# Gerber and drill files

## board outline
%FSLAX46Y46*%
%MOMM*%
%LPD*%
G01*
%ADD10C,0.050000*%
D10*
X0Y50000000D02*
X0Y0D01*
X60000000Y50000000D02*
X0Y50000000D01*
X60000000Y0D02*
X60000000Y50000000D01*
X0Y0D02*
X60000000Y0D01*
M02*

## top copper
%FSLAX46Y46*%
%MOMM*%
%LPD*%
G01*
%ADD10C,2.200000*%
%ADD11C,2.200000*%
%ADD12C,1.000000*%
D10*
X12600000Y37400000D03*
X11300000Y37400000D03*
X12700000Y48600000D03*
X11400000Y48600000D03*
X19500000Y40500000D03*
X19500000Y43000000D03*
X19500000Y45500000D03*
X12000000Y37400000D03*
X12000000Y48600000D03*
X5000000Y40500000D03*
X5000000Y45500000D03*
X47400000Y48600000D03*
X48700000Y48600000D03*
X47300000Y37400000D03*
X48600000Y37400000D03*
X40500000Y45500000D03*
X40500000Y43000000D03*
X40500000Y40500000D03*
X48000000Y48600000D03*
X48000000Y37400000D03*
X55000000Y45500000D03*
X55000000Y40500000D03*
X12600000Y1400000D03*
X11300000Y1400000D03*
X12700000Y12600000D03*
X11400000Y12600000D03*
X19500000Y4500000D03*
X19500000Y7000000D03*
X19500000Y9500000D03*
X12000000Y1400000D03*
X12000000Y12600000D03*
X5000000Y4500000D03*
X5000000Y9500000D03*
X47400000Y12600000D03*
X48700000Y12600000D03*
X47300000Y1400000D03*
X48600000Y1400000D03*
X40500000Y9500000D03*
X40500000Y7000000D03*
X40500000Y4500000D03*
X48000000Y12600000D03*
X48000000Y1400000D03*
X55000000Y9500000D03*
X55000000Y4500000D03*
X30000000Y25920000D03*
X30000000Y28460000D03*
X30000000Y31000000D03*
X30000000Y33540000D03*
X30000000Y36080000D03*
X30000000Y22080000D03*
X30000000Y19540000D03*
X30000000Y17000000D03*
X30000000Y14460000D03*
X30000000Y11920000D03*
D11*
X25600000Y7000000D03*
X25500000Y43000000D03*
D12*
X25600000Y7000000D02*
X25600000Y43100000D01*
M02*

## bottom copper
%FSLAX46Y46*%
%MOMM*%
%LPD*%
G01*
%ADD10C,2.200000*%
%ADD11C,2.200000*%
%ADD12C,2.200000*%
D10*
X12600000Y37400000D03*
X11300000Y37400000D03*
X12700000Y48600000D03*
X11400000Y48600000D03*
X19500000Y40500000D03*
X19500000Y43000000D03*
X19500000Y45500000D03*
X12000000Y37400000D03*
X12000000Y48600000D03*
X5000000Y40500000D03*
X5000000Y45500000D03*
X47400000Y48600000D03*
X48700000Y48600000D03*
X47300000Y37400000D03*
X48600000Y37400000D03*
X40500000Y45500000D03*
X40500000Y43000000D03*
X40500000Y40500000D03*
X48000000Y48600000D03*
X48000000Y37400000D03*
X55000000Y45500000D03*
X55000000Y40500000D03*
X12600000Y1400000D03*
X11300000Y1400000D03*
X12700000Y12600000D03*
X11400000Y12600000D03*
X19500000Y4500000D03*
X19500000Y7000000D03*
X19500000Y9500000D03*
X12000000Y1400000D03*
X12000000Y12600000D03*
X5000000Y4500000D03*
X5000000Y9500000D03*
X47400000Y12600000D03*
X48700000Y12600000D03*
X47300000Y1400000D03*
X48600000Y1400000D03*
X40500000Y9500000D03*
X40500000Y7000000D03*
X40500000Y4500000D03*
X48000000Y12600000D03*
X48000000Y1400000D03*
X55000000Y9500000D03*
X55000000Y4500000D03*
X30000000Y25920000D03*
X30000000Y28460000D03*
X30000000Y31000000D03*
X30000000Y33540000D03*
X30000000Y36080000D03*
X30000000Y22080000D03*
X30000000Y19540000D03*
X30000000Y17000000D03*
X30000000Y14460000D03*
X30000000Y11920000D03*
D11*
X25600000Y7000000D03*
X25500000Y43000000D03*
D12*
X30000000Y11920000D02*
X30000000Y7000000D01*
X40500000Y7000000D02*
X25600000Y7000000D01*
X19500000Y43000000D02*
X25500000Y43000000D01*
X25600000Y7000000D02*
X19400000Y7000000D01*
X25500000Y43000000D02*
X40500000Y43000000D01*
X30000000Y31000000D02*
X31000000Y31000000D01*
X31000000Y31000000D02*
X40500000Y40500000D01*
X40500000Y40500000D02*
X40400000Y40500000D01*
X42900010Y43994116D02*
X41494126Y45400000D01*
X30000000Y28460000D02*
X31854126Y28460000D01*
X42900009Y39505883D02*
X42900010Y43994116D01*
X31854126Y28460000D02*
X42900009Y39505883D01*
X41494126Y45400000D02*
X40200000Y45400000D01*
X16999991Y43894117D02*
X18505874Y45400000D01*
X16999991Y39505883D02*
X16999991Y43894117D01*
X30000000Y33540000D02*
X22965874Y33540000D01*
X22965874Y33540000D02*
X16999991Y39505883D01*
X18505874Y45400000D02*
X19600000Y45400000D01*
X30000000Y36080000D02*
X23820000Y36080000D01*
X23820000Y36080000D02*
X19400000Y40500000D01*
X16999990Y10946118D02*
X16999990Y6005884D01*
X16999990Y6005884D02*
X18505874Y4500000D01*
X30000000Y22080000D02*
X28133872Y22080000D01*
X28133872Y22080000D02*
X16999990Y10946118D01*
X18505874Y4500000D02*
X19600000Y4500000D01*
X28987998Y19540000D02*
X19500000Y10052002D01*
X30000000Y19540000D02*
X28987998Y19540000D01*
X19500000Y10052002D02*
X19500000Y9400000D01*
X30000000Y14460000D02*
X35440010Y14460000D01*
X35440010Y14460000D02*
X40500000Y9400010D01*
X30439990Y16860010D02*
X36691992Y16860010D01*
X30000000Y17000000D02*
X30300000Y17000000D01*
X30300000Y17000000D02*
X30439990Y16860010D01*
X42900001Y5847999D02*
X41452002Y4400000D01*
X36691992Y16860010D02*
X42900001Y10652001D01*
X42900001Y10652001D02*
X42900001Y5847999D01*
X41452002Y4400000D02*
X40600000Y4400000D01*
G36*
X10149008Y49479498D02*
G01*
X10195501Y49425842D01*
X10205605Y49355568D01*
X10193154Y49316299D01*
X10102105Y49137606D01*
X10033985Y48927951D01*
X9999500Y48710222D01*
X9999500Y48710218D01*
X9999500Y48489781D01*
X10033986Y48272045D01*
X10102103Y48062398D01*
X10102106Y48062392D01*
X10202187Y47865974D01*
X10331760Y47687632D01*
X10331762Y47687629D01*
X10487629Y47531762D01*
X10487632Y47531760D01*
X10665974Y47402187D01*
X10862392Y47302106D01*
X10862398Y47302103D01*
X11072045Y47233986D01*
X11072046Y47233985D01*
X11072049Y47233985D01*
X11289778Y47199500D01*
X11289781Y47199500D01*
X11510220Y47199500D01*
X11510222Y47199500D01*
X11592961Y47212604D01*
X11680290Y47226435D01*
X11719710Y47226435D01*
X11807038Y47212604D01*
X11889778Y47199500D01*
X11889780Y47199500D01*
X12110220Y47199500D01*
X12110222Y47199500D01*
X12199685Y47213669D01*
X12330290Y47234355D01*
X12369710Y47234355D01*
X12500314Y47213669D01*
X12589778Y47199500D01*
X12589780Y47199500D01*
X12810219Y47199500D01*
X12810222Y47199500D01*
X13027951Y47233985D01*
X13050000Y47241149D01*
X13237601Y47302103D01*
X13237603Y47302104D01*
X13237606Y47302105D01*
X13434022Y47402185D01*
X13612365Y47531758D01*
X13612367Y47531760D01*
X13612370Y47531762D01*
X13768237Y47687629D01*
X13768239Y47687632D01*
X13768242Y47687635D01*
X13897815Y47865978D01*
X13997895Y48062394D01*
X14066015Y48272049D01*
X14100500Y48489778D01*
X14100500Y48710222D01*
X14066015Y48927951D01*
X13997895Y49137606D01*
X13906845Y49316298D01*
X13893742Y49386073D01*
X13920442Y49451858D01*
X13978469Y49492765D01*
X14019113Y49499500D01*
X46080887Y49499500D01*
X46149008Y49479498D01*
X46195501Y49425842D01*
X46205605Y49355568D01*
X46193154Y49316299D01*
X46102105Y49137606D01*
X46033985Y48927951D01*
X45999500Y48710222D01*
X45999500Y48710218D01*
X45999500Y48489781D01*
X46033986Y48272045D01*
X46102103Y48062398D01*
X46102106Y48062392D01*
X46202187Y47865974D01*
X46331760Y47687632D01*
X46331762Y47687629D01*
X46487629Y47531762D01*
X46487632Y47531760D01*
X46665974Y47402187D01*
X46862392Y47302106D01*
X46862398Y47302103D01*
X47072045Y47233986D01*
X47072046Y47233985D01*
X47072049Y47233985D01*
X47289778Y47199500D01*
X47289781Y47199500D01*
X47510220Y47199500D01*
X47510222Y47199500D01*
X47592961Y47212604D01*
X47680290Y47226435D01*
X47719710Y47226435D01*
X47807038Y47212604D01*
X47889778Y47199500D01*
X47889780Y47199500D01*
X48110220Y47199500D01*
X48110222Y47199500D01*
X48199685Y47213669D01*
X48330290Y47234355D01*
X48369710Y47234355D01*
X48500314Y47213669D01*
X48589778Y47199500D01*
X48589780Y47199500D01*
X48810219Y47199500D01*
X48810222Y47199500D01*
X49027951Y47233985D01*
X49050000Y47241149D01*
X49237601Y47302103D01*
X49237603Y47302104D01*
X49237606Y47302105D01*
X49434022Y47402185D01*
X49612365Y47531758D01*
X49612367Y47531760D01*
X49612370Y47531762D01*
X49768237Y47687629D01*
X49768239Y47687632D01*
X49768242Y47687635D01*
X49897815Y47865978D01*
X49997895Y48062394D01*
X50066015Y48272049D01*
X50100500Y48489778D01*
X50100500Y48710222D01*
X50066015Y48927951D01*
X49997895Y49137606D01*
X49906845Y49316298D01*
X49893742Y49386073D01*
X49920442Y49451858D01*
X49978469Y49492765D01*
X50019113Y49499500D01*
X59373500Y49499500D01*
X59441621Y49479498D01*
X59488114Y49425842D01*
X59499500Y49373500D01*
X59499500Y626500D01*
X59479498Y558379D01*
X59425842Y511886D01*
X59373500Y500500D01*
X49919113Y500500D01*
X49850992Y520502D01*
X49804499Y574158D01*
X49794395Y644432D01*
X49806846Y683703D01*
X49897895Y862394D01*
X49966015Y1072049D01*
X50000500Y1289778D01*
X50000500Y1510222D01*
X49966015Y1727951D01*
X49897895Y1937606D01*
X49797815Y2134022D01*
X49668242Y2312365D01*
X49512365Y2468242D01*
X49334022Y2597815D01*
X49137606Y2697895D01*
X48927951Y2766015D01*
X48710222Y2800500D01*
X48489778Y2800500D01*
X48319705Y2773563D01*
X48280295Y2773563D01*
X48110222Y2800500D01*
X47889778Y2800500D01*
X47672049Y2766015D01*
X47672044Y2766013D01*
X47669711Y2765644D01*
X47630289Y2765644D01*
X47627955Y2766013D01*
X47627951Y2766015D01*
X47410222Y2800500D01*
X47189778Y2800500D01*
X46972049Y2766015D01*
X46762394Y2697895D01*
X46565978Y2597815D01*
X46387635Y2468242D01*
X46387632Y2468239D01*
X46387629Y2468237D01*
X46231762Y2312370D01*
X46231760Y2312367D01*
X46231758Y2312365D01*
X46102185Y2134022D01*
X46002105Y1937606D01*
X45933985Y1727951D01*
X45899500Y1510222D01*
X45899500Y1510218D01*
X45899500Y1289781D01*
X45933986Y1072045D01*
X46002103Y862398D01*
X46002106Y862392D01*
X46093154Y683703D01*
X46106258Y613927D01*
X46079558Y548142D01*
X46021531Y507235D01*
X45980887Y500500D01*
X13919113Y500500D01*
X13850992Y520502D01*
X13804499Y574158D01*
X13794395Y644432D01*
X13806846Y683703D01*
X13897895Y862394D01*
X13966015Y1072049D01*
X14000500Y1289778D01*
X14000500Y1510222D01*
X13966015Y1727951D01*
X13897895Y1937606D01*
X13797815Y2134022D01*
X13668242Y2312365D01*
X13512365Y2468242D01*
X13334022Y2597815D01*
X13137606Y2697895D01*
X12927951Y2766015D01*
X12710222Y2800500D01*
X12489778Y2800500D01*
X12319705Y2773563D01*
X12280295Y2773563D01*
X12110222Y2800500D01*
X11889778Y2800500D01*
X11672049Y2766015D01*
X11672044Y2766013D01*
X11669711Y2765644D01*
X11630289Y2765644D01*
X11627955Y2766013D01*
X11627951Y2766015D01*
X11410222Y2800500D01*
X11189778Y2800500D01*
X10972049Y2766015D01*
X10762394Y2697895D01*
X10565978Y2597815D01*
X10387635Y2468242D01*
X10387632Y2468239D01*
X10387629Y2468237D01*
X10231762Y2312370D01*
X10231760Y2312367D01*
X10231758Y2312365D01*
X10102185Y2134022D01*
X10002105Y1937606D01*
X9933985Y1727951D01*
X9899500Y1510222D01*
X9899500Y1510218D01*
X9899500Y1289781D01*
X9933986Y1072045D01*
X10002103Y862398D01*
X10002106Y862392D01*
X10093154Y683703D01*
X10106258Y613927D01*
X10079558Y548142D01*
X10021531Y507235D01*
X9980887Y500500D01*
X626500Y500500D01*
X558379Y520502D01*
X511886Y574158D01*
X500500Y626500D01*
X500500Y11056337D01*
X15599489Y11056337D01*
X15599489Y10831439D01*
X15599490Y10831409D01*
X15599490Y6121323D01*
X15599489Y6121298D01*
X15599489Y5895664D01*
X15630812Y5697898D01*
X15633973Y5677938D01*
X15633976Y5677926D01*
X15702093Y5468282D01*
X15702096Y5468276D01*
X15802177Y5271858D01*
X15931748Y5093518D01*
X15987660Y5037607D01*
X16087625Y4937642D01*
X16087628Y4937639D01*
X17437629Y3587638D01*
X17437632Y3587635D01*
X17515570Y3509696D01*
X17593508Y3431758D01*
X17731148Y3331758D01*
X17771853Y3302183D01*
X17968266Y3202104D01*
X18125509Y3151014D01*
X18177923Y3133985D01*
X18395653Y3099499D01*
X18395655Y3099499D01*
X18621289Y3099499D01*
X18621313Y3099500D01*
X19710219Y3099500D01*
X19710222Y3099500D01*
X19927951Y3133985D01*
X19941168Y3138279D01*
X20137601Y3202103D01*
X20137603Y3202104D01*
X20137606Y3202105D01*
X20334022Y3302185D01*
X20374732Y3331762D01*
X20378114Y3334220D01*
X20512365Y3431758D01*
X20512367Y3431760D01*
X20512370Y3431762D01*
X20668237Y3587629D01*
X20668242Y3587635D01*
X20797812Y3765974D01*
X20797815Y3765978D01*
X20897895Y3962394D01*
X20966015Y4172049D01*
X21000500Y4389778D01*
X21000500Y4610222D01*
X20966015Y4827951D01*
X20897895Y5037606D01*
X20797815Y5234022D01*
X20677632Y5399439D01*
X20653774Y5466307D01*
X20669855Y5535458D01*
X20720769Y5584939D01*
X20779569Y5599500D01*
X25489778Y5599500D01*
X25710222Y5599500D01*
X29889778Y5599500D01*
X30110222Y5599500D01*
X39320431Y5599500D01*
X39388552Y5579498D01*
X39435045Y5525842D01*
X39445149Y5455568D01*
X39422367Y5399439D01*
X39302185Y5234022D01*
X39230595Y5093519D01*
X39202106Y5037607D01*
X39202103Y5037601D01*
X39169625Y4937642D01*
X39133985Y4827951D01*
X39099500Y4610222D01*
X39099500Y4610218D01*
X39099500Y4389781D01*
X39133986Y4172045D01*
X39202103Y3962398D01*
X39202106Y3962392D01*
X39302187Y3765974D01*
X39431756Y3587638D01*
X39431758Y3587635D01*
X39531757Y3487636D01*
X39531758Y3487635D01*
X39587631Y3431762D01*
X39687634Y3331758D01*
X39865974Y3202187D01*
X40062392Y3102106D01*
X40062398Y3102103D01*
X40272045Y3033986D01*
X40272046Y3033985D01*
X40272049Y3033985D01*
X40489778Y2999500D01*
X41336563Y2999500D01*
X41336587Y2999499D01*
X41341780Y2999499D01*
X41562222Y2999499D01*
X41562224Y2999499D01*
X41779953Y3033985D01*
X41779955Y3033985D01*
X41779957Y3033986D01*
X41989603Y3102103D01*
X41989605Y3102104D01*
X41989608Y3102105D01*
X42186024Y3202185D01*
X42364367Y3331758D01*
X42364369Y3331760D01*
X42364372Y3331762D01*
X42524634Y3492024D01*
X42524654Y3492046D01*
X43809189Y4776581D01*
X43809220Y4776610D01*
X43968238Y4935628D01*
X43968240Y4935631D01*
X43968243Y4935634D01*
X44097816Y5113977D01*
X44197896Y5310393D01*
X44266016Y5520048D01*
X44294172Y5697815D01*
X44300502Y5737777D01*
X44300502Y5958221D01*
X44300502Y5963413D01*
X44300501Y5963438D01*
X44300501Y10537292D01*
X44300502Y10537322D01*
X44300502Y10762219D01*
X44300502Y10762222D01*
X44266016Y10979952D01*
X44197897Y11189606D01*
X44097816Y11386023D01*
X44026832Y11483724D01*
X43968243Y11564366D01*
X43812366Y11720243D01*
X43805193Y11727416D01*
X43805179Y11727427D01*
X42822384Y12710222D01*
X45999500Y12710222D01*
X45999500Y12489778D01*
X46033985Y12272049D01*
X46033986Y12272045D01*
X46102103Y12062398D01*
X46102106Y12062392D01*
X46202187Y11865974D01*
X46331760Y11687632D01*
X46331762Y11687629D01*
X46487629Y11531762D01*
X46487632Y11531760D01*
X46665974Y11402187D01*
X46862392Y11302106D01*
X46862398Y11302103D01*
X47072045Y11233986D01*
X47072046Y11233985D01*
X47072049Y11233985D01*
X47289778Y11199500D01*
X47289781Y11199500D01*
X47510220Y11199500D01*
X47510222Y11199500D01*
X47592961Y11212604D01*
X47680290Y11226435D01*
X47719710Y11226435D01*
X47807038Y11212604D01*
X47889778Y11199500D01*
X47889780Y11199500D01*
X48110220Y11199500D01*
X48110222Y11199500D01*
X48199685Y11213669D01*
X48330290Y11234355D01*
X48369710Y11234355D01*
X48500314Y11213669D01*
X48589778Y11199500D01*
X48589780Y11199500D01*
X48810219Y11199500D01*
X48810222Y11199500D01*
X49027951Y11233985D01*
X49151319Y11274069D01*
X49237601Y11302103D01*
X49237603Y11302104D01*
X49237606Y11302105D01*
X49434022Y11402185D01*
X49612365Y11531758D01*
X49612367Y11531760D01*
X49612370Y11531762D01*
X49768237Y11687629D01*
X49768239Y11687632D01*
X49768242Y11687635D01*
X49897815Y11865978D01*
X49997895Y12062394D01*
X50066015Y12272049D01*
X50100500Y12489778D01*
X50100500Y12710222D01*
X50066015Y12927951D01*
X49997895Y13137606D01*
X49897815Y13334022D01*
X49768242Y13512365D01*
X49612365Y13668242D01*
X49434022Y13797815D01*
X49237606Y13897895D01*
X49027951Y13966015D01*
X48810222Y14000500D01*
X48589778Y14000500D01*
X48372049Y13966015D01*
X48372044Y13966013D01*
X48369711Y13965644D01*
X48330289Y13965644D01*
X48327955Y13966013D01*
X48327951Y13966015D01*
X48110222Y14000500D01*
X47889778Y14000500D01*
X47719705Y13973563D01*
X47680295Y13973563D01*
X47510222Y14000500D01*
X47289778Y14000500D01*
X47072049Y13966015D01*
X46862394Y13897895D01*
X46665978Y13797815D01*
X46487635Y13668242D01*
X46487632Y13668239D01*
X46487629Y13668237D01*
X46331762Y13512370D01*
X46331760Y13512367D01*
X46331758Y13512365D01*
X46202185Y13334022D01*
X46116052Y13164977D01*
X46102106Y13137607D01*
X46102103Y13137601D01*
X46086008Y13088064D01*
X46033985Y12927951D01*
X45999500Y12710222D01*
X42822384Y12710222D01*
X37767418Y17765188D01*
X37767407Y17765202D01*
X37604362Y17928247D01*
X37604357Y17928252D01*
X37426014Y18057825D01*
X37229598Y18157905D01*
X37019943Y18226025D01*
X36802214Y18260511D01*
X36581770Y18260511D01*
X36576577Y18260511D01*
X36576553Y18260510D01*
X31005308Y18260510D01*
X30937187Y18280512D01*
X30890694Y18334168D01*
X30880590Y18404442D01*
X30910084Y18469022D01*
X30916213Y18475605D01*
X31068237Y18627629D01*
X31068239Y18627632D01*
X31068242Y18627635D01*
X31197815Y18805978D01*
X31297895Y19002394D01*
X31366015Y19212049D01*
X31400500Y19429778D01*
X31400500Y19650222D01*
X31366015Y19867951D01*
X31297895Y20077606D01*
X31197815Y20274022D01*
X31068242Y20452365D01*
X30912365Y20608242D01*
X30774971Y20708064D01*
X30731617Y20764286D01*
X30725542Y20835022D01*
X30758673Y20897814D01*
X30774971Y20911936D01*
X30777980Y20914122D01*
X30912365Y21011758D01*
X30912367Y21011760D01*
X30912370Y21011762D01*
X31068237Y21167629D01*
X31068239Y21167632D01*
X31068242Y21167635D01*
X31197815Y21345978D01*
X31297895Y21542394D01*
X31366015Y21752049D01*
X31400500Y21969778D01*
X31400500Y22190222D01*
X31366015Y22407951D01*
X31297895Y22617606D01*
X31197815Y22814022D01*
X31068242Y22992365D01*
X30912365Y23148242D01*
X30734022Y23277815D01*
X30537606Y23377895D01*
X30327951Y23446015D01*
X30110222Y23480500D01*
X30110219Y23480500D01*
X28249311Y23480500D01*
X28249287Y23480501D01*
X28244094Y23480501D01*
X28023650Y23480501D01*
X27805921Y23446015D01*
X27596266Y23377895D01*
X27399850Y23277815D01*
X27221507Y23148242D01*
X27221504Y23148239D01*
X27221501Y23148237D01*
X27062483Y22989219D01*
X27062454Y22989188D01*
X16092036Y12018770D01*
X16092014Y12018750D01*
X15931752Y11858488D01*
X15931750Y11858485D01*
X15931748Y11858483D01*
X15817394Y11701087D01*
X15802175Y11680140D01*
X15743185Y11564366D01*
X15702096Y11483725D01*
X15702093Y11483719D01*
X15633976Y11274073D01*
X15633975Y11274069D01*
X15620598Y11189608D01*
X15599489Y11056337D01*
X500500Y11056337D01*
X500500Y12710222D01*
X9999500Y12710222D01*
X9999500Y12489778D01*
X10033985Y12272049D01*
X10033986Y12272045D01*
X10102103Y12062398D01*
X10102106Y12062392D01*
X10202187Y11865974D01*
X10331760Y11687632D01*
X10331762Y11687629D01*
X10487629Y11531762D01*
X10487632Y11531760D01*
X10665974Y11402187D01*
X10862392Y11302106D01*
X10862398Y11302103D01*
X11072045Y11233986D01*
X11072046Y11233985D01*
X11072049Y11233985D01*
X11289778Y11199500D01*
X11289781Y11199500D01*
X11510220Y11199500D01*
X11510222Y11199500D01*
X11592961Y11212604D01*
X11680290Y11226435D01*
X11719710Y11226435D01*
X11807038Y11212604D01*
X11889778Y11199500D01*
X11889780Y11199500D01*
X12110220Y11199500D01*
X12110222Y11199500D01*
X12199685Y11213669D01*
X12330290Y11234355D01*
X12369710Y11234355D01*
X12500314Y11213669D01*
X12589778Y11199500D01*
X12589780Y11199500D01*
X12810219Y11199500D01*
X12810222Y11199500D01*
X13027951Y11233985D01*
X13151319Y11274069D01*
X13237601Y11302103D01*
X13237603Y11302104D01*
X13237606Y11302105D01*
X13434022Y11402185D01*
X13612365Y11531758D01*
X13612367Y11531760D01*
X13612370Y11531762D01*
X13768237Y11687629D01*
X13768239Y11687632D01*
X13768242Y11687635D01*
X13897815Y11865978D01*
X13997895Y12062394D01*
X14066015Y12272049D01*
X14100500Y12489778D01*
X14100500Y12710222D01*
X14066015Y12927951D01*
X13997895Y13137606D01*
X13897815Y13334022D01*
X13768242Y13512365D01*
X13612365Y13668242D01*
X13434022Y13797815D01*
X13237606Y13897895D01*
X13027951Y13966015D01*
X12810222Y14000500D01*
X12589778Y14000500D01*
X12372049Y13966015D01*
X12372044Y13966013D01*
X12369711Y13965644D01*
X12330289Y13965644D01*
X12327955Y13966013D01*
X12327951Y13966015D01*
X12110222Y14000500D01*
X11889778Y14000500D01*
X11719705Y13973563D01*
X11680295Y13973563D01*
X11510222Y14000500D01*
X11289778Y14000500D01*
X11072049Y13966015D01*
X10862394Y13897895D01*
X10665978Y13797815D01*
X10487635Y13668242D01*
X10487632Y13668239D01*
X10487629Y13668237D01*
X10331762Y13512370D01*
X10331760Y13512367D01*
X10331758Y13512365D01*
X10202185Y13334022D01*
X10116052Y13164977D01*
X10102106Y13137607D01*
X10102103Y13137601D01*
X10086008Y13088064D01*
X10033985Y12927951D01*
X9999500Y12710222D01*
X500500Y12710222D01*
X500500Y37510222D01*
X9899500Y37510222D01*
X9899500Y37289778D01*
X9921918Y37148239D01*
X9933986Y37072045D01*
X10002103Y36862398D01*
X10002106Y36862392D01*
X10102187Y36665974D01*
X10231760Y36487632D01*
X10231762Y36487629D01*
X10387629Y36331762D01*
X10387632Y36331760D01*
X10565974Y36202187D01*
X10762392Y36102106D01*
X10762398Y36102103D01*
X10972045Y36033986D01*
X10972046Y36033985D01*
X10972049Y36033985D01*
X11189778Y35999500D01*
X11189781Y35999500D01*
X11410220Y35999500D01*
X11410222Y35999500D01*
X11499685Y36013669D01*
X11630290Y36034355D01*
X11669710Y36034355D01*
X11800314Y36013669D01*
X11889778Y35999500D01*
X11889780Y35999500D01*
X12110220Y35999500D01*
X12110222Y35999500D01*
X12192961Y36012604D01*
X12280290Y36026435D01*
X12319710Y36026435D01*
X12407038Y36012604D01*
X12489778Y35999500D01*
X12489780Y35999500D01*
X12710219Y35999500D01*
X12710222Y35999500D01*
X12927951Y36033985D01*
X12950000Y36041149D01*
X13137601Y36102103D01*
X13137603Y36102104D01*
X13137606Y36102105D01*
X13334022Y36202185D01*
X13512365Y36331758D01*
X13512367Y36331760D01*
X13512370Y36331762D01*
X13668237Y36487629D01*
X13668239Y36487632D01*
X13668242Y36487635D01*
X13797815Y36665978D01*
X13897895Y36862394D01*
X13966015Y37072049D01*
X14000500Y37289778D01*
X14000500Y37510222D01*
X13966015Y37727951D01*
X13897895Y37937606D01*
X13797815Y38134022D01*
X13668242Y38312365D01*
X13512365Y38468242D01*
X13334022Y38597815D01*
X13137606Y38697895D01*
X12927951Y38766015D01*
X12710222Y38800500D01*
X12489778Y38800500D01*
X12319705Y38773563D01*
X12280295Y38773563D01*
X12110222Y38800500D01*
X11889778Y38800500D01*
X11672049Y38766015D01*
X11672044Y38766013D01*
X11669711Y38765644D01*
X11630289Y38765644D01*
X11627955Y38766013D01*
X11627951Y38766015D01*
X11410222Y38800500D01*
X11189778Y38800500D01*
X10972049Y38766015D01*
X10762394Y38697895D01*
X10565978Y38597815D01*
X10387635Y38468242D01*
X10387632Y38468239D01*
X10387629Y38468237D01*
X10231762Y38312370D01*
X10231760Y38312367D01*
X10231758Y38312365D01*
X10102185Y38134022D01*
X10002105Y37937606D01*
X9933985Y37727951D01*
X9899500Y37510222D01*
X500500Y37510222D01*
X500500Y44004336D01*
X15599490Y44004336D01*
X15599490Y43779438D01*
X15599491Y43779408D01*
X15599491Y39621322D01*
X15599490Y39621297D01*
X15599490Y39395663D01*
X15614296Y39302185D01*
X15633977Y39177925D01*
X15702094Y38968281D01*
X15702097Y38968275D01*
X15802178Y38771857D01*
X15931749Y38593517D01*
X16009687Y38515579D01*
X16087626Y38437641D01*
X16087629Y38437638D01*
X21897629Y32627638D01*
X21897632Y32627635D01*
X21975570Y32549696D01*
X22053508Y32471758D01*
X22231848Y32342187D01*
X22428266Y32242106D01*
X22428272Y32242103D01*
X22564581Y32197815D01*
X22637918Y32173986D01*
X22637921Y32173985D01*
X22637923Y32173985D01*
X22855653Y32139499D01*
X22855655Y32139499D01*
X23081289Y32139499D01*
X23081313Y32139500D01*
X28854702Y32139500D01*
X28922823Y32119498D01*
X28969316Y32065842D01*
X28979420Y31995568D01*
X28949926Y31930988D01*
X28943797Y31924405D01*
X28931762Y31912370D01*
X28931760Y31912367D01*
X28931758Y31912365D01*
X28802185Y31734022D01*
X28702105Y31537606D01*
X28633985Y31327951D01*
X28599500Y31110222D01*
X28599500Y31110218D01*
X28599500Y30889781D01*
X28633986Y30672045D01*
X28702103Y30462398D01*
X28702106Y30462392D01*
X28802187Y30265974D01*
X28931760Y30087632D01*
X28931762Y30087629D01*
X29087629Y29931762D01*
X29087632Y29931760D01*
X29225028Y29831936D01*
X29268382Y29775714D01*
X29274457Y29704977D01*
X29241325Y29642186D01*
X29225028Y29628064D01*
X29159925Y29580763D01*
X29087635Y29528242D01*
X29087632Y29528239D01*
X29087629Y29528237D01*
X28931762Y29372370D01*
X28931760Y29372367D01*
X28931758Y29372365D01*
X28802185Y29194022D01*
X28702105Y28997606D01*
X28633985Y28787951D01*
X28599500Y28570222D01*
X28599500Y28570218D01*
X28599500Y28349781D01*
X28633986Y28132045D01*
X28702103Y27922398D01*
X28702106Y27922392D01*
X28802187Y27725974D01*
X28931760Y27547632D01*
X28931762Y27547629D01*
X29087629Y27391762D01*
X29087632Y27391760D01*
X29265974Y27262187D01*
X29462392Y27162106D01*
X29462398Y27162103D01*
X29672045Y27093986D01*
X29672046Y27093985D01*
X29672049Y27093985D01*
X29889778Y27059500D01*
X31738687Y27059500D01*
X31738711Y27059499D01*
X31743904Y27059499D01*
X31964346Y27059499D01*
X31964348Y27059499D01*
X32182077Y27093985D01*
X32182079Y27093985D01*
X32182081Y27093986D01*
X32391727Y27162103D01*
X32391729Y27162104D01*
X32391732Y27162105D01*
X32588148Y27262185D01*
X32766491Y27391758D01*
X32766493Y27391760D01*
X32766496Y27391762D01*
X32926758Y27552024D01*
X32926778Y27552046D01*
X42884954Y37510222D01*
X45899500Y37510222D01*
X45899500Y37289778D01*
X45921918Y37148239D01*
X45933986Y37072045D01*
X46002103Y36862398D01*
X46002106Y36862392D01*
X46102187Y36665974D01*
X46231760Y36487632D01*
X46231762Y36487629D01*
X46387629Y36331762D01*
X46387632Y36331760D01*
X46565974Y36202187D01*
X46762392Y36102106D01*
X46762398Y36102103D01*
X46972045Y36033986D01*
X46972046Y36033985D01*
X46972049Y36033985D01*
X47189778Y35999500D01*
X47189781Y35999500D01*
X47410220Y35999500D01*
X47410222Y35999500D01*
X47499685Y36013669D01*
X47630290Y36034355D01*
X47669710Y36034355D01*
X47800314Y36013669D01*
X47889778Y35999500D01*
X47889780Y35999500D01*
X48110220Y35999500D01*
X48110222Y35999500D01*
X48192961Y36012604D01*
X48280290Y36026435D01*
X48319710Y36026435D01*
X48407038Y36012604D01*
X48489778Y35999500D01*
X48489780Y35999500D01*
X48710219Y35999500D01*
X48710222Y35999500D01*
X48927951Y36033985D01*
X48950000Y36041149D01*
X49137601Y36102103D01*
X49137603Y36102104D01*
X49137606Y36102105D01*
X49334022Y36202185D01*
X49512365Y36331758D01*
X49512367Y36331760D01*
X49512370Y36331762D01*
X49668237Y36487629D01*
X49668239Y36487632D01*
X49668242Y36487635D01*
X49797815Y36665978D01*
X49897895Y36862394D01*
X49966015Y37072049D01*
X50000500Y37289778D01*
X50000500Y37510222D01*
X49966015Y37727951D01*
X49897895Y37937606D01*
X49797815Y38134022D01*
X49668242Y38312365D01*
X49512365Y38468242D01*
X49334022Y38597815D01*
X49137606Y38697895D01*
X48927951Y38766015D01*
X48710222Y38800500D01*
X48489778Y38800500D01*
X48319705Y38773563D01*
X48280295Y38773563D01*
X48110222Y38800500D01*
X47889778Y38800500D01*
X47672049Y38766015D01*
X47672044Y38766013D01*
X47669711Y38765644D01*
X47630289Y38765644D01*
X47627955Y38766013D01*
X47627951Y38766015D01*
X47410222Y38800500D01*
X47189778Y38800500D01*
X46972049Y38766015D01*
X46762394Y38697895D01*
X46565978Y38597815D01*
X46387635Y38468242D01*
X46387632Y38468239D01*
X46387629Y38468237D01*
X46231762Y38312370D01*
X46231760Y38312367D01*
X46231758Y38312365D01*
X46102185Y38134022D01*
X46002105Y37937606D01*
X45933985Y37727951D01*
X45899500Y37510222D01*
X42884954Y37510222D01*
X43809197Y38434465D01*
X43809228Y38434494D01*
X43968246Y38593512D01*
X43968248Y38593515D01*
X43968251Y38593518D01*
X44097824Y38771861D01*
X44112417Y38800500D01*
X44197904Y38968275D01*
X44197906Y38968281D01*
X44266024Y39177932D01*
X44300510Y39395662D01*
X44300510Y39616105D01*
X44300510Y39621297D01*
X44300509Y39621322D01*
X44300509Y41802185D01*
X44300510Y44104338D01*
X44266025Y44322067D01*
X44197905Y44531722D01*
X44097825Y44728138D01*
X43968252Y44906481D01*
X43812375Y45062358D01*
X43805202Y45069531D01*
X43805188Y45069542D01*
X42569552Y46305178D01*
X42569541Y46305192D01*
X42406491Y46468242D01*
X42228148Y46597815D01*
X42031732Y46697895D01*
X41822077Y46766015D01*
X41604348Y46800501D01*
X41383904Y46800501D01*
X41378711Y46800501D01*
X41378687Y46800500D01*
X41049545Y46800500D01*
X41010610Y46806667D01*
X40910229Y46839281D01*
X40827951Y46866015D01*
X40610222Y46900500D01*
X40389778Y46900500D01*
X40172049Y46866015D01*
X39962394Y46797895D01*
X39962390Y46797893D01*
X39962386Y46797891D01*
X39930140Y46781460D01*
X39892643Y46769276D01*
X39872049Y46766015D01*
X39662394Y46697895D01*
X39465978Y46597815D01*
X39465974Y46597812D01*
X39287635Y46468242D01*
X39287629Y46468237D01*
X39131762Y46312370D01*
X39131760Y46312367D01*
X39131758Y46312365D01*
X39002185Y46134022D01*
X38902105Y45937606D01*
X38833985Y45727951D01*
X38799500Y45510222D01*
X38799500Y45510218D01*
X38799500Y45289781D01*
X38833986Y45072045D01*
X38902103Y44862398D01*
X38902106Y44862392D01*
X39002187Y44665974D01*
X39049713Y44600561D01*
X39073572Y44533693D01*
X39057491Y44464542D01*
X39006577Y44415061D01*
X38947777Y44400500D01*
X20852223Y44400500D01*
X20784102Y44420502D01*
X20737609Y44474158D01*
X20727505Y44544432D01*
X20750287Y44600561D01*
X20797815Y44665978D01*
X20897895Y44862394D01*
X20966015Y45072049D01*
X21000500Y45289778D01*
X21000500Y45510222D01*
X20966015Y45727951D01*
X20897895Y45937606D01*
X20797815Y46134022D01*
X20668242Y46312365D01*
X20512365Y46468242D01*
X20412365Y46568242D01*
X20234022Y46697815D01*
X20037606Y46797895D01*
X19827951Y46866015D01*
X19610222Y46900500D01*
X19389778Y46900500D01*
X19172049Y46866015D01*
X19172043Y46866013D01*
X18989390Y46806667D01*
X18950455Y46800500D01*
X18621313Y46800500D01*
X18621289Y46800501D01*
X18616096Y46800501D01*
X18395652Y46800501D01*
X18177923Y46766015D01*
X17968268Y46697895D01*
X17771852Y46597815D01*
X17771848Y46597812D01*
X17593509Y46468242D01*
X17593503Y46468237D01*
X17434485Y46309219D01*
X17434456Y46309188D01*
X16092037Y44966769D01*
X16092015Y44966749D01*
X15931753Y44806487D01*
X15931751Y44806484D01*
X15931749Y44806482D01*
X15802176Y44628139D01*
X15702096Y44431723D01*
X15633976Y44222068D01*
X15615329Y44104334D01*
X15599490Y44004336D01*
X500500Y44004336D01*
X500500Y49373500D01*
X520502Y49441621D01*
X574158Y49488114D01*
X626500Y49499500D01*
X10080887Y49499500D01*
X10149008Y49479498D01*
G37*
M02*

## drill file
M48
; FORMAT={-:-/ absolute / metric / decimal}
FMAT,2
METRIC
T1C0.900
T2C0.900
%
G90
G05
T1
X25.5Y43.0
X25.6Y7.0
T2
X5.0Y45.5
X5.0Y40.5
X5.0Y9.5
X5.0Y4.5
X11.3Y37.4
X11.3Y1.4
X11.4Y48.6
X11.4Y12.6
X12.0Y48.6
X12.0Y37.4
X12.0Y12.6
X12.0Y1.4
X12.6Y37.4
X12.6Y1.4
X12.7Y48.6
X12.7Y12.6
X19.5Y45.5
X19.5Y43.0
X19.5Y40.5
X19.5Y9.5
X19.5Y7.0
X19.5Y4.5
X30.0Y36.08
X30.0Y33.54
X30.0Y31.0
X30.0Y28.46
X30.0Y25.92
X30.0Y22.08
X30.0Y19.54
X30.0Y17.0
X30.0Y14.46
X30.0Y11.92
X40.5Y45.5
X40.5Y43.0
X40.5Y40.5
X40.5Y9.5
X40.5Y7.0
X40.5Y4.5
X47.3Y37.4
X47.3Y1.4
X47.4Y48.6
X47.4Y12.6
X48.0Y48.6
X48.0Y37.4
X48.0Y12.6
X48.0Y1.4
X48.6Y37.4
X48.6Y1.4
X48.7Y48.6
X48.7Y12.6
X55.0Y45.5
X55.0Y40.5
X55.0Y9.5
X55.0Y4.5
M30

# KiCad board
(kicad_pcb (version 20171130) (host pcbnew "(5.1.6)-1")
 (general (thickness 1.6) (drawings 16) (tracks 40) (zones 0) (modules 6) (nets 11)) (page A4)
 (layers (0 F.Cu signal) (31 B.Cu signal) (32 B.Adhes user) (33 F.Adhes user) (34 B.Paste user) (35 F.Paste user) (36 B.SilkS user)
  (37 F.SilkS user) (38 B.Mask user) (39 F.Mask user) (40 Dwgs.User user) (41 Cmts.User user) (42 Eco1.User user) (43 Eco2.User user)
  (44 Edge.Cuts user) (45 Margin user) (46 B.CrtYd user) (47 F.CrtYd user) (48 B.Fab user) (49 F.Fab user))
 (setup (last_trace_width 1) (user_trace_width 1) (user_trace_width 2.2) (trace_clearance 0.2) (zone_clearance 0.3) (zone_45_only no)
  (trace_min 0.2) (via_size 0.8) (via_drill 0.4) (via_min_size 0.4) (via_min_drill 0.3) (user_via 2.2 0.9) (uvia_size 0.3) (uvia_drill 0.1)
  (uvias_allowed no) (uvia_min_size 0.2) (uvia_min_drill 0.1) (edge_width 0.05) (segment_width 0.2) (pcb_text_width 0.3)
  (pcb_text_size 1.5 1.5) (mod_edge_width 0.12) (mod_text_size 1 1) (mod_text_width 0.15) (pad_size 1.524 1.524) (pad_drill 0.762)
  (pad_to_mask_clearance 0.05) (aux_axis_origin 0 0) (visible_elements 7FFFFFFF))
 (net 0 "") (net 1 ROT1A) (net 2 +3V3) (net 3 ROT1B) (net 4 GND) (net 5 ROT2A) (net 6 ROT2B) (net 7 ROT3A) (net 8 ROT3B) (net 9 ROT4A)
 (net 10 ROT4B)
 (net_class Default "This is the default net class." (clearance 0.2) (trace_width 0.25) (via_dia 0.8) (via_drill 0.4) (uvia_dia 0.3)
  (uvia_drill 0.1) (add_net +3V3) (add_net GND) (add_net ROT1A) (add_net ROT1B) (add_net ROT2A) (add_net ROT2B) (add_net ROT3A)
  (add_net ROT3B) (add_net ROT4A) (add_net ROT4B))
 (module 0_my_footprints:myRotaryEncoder (layer F.Cu) (at 12 -43 180)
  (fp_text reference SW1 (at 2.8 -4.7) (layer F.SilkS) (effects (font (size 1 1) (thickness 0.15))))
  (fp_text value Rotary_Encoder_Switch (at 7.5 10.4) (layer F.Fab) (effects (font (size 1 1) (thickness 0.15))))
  (pad "" thru_hole circle (at -0.6 -5.6 180) (size 2.2 2.2) (drill 0.9) (layers *.Cu *.Mask))
  (pad "" thru_hole circle (at 0.7 -5.6 180) (size 2.2 2.2) (drill 0.9) (layers *.Cu *.Mask))
  (pad "" thru_hole circle (at -0.7 5.6 180) (size 2.2 2.2) (drill 0.9) (layers *.Cu *.Mask))
  (pad "" thru_hole circle (at 0.6 5.6 180) (size 2.2 2.2) (drill 0.9) (layers *.Cu *.Mask))
  (pad A thru_hole circle (at -7.5 -2.5 180) (size 2.2 2.2) (drill 0.9) (layers *.Cu *.Mask) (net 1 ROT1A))
  (pad C thru_hole circle (at -7.5 0 180) (size 2.2 2.2) (drill 0.9) (layers *.Cu *.Mask) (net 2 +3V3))
  (pad B thru_hole circle (at -7.5 2.5 180) (size 2.2 2.2) (drill 0.9) (layers *.Cu *.Mask) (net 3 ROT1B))
  (pad "" thru_hole circle (at 0 -5.6 180) (size 2.2 2.2) (drill 0.9) (layers *.Cu *.Mask))
  (pad "" thru_hole circle (at 0 5.6 180) (size 2.2 2.2) (drill 0.9) (layers *.Cu *.Mask))
  (pad S1 thru_hole circle (at 7 -2.5 180) (size 2.2 2.2) (drill 0.9) (layers *.Cu *.Mask) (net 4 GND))
  (pad S2 thru_hole circle (at 7 2.5 180) (size 2.2 2.2) (drill 0.9) (layers *.Cu *.Mask) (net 4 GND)))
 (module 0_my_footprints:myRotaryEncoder (layer F.Cu) (at 48 -43)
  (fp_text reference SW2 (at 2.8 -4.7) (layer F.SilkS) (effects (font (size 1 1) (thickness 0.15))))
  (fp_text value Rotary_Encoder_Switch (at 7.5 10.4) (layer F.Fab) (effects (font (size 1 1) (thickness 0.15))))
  (pad "" thru_hole circle (at -0.6 -5.6) (size 2.2 2.2) (drill 0.9) (layers *.Cu *.Mask))
  (pad "" thru_hole circle (at 0.7 -5.6) (size 2.2 2.2) (drill 0.9) (layers *.Cu *.Mask))
  (pad "" thru_hole circle (at -0.7 5.6) (size 2.2 2.2) (drill 0.9) (layers *.Cu *.Mask))
  (pad "" thru_hole circle (at 0.6 5.6) (size 2.2 2.2) (drill 0.9) (layers *.Cu *.Mask))
  (pad A thru_hole circle (at -7.5 -2.5) (size 2.2 2.2) (drill 0.9) (layers *.Cu *.Mask) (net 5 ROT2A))
  (pad C thru_hole circle (at -7.5 0) (size 2.2 2.2) (drill 0.9) (layers *.Cu *.Mask) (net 2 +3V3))
  (pad B thru_hole circle (at -7.5 2.5) (size 2.2 2.2) (drill 0.9) (layers *.Cu *.Mask) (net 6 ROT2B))
  (pad "" thru_hole circle (at 0 -5.6) (size 2.2 2.2) (drill 0.9) (layers *.Cu *.Mask))
  (pad "" thru_hole circle (at 0 5.6) (size 2.2 2.2) (drill 0.9) (layers *.Cu *.Mask))
  (pad S1 thru_hole circle (at 7 -2.5) (size 2.2 2.2) (drill 0.9) (layers *.Cu *.Mask) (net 4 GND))
  (pad S2 thru_hole circle (at 7 2.5) (size 2.2 2.2) (drill 0.9) (layers *.Cu *.Mask) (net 4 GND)))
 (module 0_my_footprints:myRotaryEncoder (layer F.Cu) (at 12 -7 180)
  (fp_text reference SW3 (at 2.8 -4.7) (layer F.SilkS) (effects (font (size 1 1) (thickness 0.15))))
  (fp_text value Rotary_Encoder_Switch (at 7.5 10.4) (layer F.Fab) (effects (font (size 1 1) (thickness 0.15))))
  (pad "" thru_hole circle (at -0.6 -5.6 180) (size 2.2 2.2) (drill 0.9) (layers *.Cu *.Mask))
  (pad "" thru_hole circle (at 0.7 -5.6 180) (size 2.2 2.2) (drill 0.9) (layers *.Cu *.Mask))
  (pad "" thru_hole circle (at -0.7 5.6 180) (size 2.2 2.2) (drill 0.9) (layers *.Cu *.Mask))
  (pad "" thru_hole circle (at 0.6 5.6 180) (size 2.2 2.2) (drill 0.9) (layers *.Cu *.Mask))
  (pad A thru_hole circle (at -7.5 -2.5 180) (size 2.2 2.2) (drill 0.9) (layers *.Cu *.Mask) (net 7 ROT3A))
  (pad C thru_hole circle (at -7.5 0 180) (size 2.2 2.2) (drill 0.9) (layers *.Cu *.Mask) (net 2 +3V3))
  (pad B thru_hole circle (at -7.5 2.5 180) (size 2.2 2.2) (drill 0.9) (layers *.Cu *.Mask) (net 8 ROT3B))
  (pad "" thru_hole circle (at 0 -5.6 180) (size 2.2 2.2) (drill 0.9) (layers *.Cu *.Mask))
  (pad "" thru_hole circle (at 0 5.6 180) (size 2.2 2.2) (drill 0.9) (layers *.Cu *.Mask))
  (pad S1 thru_hole circle (at 7 -2.5 180) (size 2.2 2.2) (drill 0.9) (layers *.Cu *.Mask) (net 4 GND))
  (pad S2 thru_hole circle (at 7 2.5 180) (size 2.2 2.2) (drill 0.9) (layers *.Cu *.Mask) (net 4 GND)))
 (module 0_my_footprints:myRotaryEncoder (layer F.Cu) (at 48 -7)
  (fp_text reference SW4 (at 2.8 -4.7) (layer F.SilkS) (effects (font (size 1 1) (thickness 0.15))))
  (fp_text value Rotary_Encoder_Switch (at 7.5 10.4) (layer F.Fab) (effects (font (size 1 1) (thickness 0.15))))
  (pad "" thru_hole circle (at -0.6 -5.6) (size 2.2 2.2) (drill 0.9) (layers *.Cu *.Mask))
  (pad "" thru_hole circle (at 0.7 -5.6) (size 2.2 2.2) (drill 0.9) (layers *.Cu *.Mask))
  (pad "" thru_hole circle (at -0.7 5.6) (size 2.2 2.2) (drill 0.9) (layers *.Cu *.Mask))
  (pad "" thru_hole circle (at 0.6 5.6) (size 2.2 2.2) (drill 0.9) (layers *.Cu *.Mask))
  (pad A thru_hole circle (at -7.5 -2.5) (size 2.2 2.2) (drill 0.9) (layers *.Cu *.Mask) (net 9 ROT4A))
  (pad C thru_hole circle (at -7.5 0) (size 2.2 2.2) (drill 0.9) (layers *.Cu *.Mask) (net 2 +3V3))
  (pad B thru_hole circle (at -7.5 2.5) (size 2.2 2.2) (drill 0.9) (layers *.Cu *.Mask) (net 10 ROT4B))
  (pad "" thru_hole circle (at 0 -5.6) (size 2.2 2.2) (drill 0.9) (layers *.Cu *.Mask))
  (pad "" thru_hole circle (at 0 5.6) (size 2.2 2.2) (drill 0.9) (layers *.Cu *.Mask))
  (pad S1 thru_hole circle (at 7 -2.5) (size 2.2 2.2) (drill 0.9) (layers *.Cu *.Mask) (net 4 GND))
  (pad S2 thru_hole circle (at 7 2.5) (size 2.2 2.2) (drill 0.9) (layers *.Cu *.Mask) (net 4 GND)))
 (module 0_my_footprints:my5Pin (layer F.Cu) (at 30 -31 270)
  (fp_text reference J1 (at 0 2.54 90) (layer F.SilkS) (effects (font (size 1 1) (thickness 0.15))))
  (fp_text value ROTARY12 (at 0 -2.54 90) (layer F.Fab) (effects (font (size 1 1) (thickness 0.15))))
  (pad 5 thru_hole circle (at 5.08 0 270) (size 2.2 2.2) (drill 0.9) (layers *.Cu *.Mask) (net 4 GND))
  (pad 4 thru_hole circle (at 2.54 0 270) (size 2.2 2.2) (drill 0.9) (layers *.Cu *.Mask) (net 5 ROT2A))
  (pad 3 thru_hole circle (at 0 0 270) (size 2.2 2.2) (drill 0.9) (layers *.Cu *.Mask) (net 6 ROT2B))
  (pad 2 thru_hole circle (at -2.54 0 270) (size 2.2 2.2) (drill 0.9) (layers *.Cu *.Mask) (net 3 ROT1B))
  (pad 1 thru_hole circle (at -5.08 0 270) (size 2.2 2.2) (drill 0.9) (layers *.Cu *.Mask) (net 1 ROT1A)))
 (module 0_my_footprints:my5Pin (layer F.Cu) (at 30 -17 270)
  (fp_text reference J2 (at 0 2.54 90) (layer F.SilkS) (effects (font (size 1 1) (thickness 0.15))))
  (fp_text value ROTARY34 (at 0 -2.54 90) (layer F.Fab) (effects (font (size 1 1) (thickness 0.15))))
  (pad 1 thru_hole circle (at -5.08 0 270) (size 2.2 2.2) (drill 0.9) (layers *.Cu *.Mask) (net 7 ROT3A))
  (pad 2 thru_hole circle (at -2.54 0 270) (size 2.2 2.2) (drill 0.9) (layers *.Cu *.Mask) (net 8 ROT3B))
  (pad 3 thru_hole circle (at 0 0 270) (size 2.2 2.2) (drill 0.9) (layers *.Cu *.Mask) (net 10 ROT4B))
  (pad 4 thru_hole circle (at 2.54 0 270) (size 2.2 2.2) (drill 0.9) (layers *.Cu *.Mask) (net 9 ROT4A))
  (pad 5 thru_hole circle (at 5.08 0 270) (size 2.2 2.2) (drill 0.9) (layers *.Cu *.Mask) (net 2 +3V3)))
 (gr_line (start 0 -50) (end 0 0) (layer Edge.Cuts) (width 0.05))
 (gr_line (start 60 -50) (end 0 -50) (layer Edge.Cuts) (width 0.05))
 (gr_line (start 60 0) (end 60 -50) (layer Edge.Cuts) (width 0.05))
 (gr_line (start 0 0) (end 60 0) (layer Edge.Cuts) (width 0.05))
 (segment (start 30 -11.92) (end 30 -7) (width 2.2) (layer B.Cu) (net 2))
 (segment (start 40.5 -7) (end 25.6 -7) (width 2.2) (layer B.Cu) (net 2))
 (segment (start 19.5 -43) (end 25.5 -43) (width 2.2) (layer B.Cu) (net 2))
 (segment (start 25.6 -7) (end 19.4 -7) (width 2.2) (layer B.Cu) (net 2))
 (via (at 25.6 -7) (size 2.2) (drill 0.9) (layers F.Cu B.Cu) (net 2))
 (segment (start 25.6 -7) (end 25.6 -43.1) (width 1) (layer F.Cu) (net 2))
 (segment (start 25.5 -43) (end 40.5 -43) (width 2.2) (layer B.Cu) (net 2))
 (via (at 25.5 -43) (size 2.2) (drill 0.9) (layers F.Cu B.Cu) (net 2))
 (segment (start 30 -31) (end 31 -31) (width 2.2) (layer B.Cu) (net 6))
 (segment (start 31 -31) (end 40.5 -40.5) (width 2.2) (layer B.Cu) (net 6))
 (segment (start 40.5 -40.5) (end 40.4 -40.5) (width 2.2) (layer B.Cu) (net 6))
 (segment (start 42.90001 -43.994116) (end 41.494126 -45.4) (width 2.2) (layer B.Cu) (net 5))
 (segment (start 30 -28.46) (end 31.854126 -28.46) (width 2.2) (layer B.Cu) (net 5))
 (segment (start 42.900009 -39.505883) (end 42.90001 -43.994116) (width 2.2) (layer B.Cu) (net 5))
 (segment (start 31.854126 -28.46) (end 42.900009 -39.505883) (width 2.2) (layer B.Cu) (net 5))
 (segment (start 41.494126 -45.4) (end 40.2 -45.4) (width 2.2) (layer B.Cu) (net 5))
 (segment (start 16.999991 -43.894117) (end 18.505874 -45.4) (width 2.2) (layer B.Cu) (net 3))
 (segment (start 16.999991 -39.505883) (end 16.999991 -43.894117) (width 2.2) (layer B.Cu) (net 3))
 (segment (start 30 -33.54) (end 22.965874 -33.54) (width 2.2) (layer B.Cu) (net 3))
 (segment (start 22.965874 -33.54) (end 16.999991 -39.505883) (width 2.2) (layer B.Cu) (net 3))
 (segment (start 18.505874 -45.4) (end 19.6 -45.4) (width 2.2) (layer B.Cu) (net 3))
 (segment (start 30 -36.08) (end 23.82 -36.08) (width 2.2) (layer B.Cu) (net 1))
 (segment (start 23.82 -36.08) (end 19.4 -40.5) (width 2.2) (layer B.Cu) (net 1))
 (segment (start 16.99999 -10.946118) (end 16.99999 -6.005884) (width 2.2) (layer B.Cu) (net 7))
 (segment (start 16.99999 -6.005884) (end 18.505874 -4.5) (width 2.2) (layer B.Cu) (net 7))
 (segment (start 30 -22.08) (end 28.133872 -22.08) (width 2.2) (layer B.Cu) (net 7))
 (segment (start 28.133872 -22.08) (end 16.99999 -10.946118) (width 2.2) (layer B.Cu) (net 7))
 (segment (start 18.505874 -4.5) (end 19.6 -4.5) (width 2.2) (layer B.Cu) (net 7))
 (segment (start 28.987998 -19.54) (end 19.5 -10.052002) (width 2.2) (layer B.Cu) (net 8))
 (segment (start 30 -19.54) (end 28.987998 -19.54) (width 2.2) (layer B.Cu) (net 8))
 (segment (start 19.5 -10.052002) (end 19.5 -9.4) (width 2.2) (layer B.Cu) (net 8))
 (segment (start 30 -14.46) (end 35.44001 -14.46) (width 2.2) (layer B.Cu) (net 9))
 (segment (start 35.44001 -14.46) (end 40.5 -9.40001) (width 2.2) (layer B.Cu) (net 9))
 (segment (start 30.43999 -16.86001) (end 36.691992 -16.86001) (width 2.2) (layer B.Cu) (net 10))
 (segment (start 30 -17) (end 30.3 -17) (width 2.2) (layer B.Cu) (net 10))
 (segment (start 30.3 -17) (end 30.43999 -16.86001) (width 2.2) (layer B.Cu) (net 10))
 (segment (start 42.900001 -5.847999) (end 41.452002 -4.4) (width 2.2) (layer B.Cu) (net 10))
 (segment (start 36.691992 -16.86001) (end 42.900001 -10.652001) (width 2.2) (layer B.Cu) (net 10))
 (segment (start 42.900001 -10.652001) (end 42.900001 -5.847999) (width 2.2) (layer B.Cu) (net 10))
 (segment (start 41.452002 -4.4) (end 40.6 -4.4) (width 2.2) (layer B.Cu) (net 10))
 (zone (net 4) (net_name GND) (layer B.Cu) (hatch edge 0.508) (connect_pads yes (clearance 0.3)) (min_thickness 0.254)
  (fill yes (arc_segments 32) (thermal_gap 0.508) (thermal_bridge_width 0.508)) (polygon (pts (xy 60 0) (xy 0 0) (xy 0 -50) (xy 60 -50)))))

